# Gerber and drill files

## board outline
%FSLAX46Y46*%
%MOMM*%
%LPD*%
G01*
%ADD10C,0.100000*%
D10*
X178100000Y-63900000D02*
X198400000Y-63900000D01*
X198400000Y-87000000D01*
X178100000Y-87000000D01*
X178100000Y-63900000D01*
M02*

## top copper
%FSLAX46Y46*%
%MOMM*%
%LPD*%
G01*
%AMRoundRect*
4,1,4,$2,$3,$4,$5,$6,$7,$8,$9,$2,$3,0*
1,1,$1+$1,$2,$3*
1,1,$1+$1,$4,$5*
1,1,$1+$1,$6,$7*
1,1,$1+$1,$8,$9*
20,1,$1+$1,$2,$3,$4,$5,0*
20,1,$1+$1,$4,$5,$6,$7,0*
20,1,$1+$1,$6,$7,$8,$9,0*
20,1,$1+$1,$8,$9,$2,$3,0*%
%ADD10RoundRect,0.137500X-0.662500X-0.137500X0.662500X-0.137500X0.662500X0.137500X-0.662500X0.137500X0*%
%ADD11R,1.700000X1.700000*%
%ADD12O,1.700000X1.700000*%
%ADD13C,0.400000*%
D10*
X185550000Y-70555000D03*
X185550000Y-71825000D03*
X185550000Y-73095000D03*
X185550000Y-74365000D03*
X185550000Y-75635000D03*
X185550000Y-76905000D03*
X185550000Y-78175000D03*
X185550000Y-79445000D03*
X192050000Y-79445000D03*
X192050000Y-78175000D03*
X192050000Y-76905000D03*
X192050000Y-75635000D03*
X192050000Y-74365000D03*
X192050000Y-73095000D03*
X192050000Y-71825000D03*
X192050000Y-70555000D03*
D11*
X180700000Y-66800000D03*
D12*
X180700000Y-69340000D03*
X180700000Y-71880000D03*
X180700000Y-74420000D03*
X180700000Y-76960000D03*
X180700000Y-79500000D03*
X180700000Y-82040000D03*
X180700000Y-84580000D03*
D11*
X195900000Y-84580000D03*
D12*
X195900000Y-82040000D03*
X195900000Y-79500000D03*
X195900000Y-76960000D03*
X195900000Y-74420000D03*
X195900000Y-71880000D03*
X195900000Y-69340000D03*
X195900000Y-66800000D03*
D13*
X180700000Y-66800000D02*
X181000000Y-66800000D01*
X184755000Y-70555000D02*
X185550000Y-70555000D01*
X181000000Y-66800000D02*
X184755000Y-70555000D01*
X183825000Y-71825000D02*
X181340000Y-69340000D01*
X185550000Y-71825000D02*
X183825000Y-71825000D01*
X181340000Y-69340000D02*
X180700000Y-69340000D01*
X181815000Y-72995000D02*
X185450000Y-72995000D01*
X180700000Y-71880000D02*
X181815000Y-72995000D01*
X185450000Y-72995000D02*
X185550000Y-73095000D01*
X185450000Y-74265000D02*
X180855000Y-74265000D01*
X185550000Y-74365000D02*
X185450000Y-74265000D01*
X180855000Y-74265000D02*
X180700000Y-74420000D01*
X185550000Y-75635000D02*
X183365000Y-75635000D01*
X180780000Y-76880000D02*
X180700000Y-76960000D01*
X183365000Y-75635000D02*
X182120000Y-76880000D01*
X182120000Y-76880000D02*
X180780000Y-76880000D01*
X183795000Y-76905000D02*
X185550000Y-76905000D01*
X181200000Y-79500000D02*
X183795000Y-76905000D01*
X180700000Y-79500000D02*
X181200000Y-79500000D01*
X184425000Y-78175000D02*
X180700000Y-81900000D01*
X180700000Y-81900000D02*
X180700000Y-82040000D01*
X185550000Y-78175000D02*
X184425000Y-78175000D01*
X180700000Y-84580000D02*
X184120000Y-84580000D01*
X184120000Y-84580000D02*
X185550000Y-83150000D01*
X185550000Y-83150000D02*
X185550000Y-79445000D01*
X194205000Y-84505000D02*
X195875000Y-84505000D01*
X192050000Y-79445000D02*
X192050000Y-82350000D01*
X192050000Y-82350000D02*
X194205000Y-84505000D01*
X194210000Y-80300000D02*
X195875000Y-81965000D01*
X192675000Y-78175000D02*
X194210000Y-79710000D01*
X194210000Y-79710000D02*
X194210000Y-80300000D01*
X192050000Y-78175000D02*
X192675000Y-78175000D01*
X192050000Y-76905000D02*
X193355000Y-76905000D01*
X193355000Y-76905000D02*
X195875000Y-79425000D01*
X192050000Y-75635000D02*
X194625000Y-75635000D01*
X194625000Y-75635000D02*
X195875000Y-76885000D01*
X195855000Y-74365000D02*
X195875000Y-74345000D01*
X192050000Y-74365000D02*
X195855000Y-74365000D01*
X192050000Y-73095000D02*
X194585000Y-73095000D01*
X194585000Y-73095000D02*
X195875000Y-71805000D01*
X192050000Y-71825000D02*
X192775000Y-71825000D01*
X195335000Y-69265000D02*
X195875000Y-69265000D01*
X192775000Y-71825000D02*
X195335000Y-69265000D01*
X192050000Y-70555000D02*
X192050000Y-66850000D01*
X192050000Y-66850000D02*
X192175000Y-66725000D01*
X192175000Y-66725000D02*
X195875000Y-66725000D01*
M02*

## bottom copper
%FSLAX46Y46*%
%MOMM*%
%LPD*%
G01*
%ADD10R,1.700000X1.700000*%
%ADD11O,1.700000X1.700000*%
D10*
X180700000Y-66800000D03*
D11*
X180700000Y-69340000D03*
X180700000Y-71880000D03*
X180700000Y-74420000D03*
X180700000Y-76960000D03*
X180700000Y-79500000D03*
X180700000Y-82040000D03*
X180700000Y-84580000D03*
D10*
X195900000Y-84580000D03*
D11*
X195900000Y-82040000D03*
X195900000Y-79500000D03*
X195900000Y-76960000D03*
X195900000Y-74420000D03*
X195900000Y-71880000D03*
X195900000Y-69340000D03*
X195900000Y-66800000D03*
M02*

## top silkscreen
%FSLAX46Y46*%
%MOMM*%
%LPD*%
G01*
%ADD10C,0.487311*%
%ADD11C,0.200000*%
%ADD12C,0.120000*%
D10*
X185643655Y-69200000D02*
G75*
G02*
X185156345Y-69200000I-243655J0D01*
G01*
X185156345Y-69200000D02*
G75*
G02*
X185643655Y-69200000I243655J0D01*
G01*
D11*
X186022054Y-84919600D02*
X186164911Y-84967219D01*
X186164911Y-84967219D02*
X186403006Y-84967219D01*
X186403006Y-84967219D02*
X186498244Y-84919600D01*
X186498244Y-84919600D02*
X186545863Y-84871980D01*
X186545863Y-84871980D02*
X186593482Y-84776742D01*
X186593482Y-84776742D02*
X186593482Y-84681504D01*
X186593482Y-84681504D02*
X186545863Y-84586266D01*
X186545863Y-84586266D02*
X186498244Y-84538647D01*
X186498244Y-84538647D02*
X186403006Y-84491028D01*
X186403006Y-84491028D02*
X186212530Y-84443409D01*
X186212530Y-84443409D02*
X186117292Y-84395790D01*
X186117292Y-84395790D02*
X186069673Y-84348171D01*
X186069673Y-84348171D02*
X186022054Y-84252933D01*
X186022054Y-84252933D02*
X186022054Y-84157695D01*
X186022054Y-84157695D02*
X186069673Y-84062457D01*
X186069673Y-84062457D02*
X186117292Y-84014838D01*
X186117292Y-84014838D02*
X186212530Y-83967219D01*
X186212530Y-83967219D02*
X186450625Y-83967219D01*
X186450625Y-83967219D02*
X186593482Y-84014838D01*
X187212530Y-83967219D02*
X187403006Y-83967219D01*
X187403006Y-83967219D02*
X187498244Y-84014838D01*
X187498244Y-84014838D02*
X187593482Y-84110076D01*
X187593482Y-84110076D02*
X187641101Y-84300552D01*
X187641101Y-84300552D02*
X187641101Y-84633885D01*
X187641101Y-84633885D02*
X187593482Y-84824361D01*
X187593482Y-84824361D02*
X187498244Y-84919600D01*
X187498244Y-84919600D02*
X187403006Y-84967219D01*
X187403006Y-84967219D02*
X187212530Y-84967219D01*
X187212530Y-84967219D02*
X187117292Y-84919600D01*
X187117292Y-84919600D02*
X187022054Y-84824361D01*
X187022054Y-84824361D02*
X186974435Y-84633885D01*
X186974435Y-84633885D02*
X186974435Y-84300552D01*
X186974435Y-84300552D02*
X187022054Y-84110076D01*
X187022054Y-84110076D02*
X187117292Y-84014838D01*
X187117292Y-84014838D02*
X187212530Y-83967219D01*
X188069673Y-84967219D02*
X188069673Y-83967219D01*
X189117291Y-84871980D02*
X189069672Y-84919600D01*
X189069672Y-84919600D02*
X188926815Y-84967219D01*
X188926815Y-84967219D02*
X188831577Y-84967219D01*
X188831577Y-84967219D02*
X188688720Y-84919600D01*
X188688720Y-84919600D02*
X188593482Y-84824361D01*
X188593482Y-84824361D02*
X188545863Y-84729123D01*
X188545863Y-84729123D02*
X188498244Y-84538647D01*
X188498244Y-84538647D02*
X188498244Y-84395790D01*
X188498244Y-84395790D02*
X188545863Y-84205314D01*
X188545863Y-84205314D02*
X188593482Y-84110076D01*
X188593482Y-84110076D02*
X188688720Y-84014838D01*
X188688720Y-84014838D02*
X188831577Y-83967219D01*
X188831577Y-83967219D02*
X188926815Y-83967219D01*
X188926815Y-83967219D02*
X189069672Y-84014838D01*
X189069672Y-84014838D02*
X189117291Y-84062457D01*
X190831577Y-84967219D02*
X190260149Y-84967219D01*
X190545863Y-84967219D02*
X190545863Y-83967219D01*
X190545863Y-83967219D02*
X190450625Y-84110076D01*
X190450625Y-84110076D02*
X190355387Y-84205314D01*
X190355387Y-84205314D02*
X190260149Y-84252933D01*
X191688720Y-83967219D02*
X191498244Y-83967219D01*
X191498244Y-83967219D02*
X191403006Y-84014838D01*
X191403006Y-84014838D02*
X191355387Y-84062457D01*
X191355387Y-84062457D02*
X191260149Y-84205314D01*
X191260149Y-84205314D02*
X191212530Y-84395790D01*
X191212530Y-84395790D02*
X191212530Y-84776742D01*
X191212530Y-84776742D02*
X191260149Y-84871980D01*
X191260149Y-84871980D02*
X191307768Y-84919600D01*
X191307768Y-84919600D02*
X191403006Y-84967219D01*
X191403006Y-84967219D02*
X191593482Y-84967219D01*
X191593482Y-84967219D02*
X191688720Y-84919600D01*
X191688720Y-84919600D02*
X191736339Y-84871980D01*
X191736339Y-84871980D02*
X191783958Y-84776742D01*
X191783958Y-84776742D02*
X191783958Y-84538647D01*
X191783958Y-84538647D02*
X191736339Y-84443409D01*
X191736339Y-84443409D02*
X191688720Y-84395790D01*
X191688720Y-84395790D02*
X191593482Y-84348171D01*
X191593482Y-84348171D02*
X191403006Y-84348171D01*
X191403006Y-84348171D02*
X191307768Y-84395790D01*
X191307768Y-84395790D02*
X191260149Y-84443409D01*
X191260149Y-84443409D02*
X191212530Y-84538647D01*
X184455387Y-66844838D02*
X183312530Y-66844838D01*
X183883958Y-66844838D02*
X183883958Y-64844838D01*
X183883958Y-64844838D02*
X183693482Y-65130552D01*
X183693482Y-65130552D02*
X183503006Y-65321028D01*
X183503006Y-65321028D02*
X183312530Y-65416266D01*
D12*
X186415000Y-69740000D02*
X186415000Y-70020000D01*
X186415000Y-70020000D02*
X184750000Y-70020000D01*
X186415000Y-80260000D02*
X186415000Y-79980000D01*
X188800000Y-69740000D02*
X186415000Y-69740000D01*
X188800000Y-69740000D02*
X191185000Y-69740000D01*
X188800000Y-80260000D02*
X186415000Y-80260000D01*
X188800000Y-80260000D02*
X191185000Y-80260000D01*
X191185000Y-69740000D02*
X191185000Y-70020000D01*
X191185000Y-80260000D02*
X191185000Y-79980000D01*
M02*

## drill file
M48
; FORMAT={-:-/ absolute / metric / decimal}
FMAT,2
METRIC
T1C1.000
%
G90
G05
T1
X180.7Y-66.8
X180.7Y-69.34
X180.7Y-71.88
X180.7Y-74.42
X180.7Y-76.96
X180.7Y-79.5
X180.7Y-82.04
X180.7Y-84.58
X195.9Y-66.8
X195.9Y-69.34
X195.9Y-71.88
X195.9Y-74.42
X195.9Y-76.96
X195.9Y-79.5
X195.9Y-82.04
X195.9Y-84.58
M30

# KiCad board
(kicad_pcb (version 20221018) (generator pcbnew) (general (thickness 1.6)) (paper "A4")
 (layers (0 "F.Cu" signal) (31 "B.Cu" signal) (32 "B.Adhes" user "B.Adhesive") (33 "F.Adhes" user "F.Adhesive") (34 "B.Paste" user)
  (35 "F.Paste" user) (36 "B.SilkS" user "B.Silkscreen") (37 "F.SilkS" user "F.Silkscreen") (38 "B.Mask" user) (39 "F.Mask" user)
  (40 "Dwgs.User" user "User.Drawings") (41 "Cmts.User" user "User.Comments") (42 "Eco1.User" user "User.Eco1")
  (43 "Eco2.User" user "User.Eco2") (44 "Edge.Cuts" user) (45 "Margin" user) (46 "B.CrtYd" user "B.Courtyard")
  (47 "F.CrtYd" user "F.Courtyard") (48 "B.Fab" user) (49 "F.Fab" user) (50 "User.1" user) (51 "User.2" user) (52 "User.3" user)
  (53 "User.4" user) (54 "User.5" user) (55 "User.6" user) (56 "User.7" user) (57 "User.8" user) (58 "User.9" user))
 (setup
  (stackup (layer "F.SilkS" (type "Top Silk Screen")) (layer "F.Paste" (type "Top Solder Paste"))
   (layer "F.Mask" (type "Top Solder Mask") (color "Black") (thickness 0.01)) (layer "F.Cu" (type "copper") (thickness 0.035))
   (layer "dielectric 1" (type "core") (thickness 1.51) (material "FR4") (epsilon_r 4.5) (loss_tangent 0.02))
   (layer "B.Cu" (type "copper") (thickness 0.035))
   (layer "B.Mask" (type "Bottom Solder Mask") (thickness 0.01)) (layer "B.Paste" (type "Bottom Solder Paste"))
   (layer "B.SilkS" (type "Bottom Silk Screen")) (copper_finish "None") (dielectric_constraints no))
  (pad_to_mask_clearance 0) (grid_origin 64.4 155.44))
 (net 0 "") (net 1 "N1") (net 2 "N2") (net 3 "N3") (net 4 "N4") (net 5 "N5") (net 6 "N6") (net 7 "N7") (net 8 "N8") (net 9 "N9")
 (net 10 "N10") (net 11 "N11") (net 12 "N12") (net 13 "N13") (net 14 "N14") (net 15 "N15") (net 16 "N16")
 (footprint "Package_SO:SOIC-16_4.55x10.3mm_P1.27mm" (layer "F.Cu") (at 188.8 75)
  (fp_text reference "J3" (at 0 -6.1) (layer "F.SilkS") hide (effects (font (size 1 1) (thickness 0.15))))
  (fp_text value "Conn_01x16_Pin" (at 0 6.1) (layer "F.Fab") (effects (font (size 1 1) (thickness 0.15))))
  (fp_line (start -2.385 -5.26) (end -2.385 -4.98) (stroke (width 0.12) (type solid)) (layer "F.SilkS"))
  (fp_line (start -2.385 -4.98) (end -4.05 -4.98) (stroke (width 0.12) (type solid)) (layer "F.SilkS"))
  (fp_line (start -2.385 5.26) (end -2.385 4.98) (stroke (width 0.12) (type solid)) (layer "F.SilkS"))
  (fp_line (start 0 -5.26) (end -2.385 -5.26) (stroke (width 0.12) (type solid)) (layer "F.SilkS"))
  (fp_line (start 0 -5.26) (end 2.385 -5.26) (stroke (width 0.12) (type solid)) (layer "F.SilkS"))
  (fp_line (start 0 5.26) (end -2.385 5.26) (stroke (width 0.12) (type solid)) (layer "F.SilkS"))
  (fp_line (start 0 5.26) (end 2.385 5.26) (stroke (width 0.12) (type solid)) (layer "F.SilkS"))
  (fp_line (start 2.385 -5.26) (end 2.385 -4.98) (stroke (width 0.12) (type solid)) (layer "F.SilkS"))
  (fp_line (start 2.385 5.26) (end 2.385 4.98) (stroke (width 0.12) (type solid)) (layer "F.SilkS"))
  (pad "1" smd roundrect (at -3.25 -4.445) (size 1.6 0.55) (layers "F.Cu" "F.Paste" "F.Mask") (roundrect_rratio 0.25) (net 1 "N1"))
  (pad "2" smd roundrect (at -3.25 -3.175) (size 1.6 0.55) (layers "F.Cu" "F.Paste" "F.Mask") (roundrect_rratio 0.25) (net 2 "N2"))
  (pad "3" smd roundrect (at -3.25 -1.905) (size 1.6 0.55) (layers "F.Cu" "F.Paste" "F.Mask") (roundrect_rratio 0.25) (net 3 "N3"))
  (pad "4" smd roundrect (at -3.25 -0.635) (size 1.6 0.55) (layers "F.Cu" "F.Paste" "F.Mask") (roundrect_rratio 0.25) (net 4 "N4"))
  (pad "5" smd roundrect (at -3.25 0.635) (size 1.6 0.55) (layers "F.Cu" "F.Paste" "F.Mask") (roundrect_rratio 0.25) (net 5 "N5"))
  (pad "6" smd roundrect (at -3.25 1.905) (size 1.6 0.55) (layers "F.Cu" "F.Paste" "F.Mask") (roundrect_rratio 0.25) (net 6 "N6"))
  (pad "7" smd roundrect (at -3.25 3.175) (size 1.6 0.55) (layers "F.Cu" "F.Paste" "F.Mask") (roundrect_rratio 0.25) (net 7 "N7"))
  (pad "8" smd roundrect (at -3.25 4.445) (size 1.6 0.55) (layers "F.Cu" "F.Paste" "F.Mask") (roundrect_rratio 0.25) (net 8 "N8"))
  (pad "9" smd roundrect (at 3.25 4.445) (size 1.6 0.55) (layers "F.Cu" "F.Paste" "F.Mask") (roundrect_rratio 0.25) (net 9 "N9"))
  (pad "10" smd roundrect (at 3.25 3.175) (size 1.6 0.55) (layers "F.Cu" "F.Paste" "F.Mask") (roundrect_rratio 0.25) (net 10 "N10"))
  (pad "11" smd roundrect (at 3.25 1.905) (size 1.6 0.55) (layers "F.Cu" "F.Paste" "F.Mask") (roundrect_rratio 0.25) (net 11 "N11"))
  (pad "12" smd roundrect (at 3.25 0.635) (size 1.6 0.55) (layers "F.Cu" "F.Paste" "F.Mask") (roundrect_rratio 0.25) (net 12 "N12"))
  (pad "13" smd roundrect (at 3.25 -0.635) (size 1.6 0.55) (layers "F.Cu" "F.Paste" "F.Mask") (roundrect_rratio 0.25) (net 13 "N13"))
  (pad "14" smd roundrect (at 3.25 -1.905) (size 1.6 0.55) (layers "F.Cu" "F.Paste" "F.Mask") (roundrect_rratio 0.25) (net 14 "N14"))
  (pad "15" smd roundrect (at 3.25 -3.175) (size 1.6 0.55) (layers "F.Cu" "F.Paste" "F.Mask") (roundrect_rratio 0.25) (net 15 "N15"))
  (pad "16" smd roundrect (at 3.25 -4.445) (size 1.6 0.55) (layers "F.Cu" "F.Paste" "F.Mask") (roundrect_rratio 0.25) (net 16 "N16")))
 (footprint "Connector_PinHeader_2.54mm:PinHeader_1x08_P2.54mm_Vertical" (layer "B.Cu") (at 180.7 66.8 180)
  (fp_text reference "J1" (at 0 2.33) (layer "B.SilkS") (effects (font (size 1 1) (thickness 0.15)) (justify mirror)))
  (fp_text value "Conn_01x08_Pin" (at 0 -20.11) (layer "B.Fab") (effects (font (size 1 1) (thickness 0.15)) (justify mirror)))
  (pad "1" thru_hole rect (at 0 0 180) (size 1.7 1.7) (drill 1) (layers "*.Cu" "*.Mask") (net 1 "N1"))
  (pad "2" thru_hole oval (at 0 -2.54 180) (size 1.7 1.7) (drill 1) (layers "*.Cu" "*.Mask") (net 2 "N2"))
  (pad "3" thru_hole oval (at 0 -5.08 180) (size 1.7 1.7) (drill 1) (layers "*.Cu" "*.Mask") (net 3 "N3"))
  (pad "4" thru_hole oval (at 0 -7.62 180) (size 1.7 1.7) (drill 1) (layers "*.Cu" "*.Mask") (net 4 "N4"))
  (pad "5" thru_hole oval (at 0 -10.16 180) (size 1.7 1.7) (drill 1) (layers "*.Cu" "*.Mask") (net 5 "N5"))
  (pad "6" thru_hole oval (at 0 -12.7 180) (size 1.7 1.7) (drill 1) (layers "*.Cu" "*.Mask") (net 6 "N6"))
  (pad "7" thru_hole oval (at 0 -15.24 180) (size 1.7 1.7) (drill 1) (layers "*.Cu" "*.Mask") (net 7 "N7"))
  (pad "8" thru_hole oval (at 0 -17.78 180) (size 1.7 1.7) (drill 1) (layers "*.Cu" "*.Mask") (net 8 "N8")))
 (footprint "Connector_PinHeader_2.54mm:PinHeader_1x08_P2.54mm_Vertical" (layer "B.Cu") (at 195.9 84.58)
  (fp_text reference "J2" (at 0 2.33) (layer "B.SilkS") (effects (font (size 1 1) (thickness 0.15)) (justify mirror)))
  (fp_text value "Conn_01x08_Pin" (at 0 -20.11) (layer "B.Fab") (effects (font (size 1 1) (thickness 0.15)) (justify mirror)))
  (pad "1" thru_hole rect (at 0 0) (size 1.7 1.7) (drill 1) (layers "*.Cu" "*.Mask") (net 9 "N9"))
  (pad "2" thru_hole oval (at 0 -2.54) (size 1.7 1.7) (drill 1) (layers "*.Cu" "*.Mask") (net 10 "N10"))
  (pad "3" thru_hole oval (at 0 -5.08) (size 1.7 1.7) (drill 1) (layers "*.Cu" "*.Mask") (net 11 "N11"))
  (pad "4" thru_hole oval (at 0 -7.62) (size 1.7 1.7) (drill 1) (layers "*.Cu" "*.Mask") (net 12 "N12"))
  (pad "5" thru_hole oval (at 0 -10.16) (size 1.7 1.7) (drill 1) (layers "*.Cu" "*.Mask") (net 13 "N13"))
  (pad "6" thru_hole oval (at 0 -12.7) (size 1.7 1.7) (drill 1) (layers "*.Cu" "*.Mask") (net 14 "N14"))
  (pad "7" thru_hole oval (at 0 -15.24) (size 1.7 1.7) (drill 1) (layers "*.Cu" "*.Mask") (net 15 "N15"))
  (pad "8" thru_hole oval (at 0 -17.78) (size 1.7 1.7) (drill 1) (layers "*.Cu" "*.Mask") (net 16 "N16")))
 (gr_circle (center 185.4 69.2) (end 185.812311 69.2) (stroke (width 0.15) (type solid)) (fill solid) (layer "F.SilkS"))
 (gr_rect (start 178.1 63.9) (end 198.4 87) (stroke (width 0.1) (type default)) (fill none) (layer "Edge.Cuts"))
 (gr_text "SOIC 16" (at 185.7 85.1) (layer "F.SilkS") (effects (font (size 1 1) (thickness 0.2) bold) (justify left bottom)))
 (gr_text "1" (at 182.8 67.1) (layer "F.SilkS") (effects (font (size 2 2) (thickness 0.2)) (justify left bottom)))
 (segment (start 180.7 66.8) (end 181 66.8) (width 0.4) (layer "F.Cu") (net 1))
 (segment (start 184.755 70.555) (end 185.55 70.555) (width 0.4) (layer "F.Cu") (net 1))
 (segment (start 181 66.8) (end 184.755 70.555) (width 0.4) (layer "F.Cu") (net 1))
 (segment (start 183.825 71.825) (end 181.34 69.34) (width 0.4) (layer "F.Cu") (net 2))
 (segment (start 185.55 71.825) (end 183.825 71.825) (width 0.4) (layer "F.Cu") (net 2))
 (segment (start 181.34 69.34) (end 180.7 69.34) (width 0.4) (layer "F.Cu") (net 2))
 (segment (start 181.815 72.995) (end 185.45 72.995) (width 0.4) (layer "F.Cu") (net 3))
 (segment (start 180.7 71.88) (end 181.815 72.995) (width 0.4) (layer "F.Cu") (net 3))
 (segment (start 185.45 72.995) (end 185.55 73.095) (width 0.4) (layer "F.Cu") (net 3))
 (segment (start 185.45 74.265) (end 180.855 74.265) (width 0.4) (layer "F.Cu") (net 4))
 (segment (start 185.55 74.365) (end 185.45 74.265) (width 0.4) (layer "F.Cu") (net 4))
 (segment (start 180.855 74.265) (end 180.7 74.42) (width 0.4) (layer "F.Cu") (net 4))
 (segment (start 185.55 75.635) (end 183.365 75.635) (width 0.4) (layer "F.Cu") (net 5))
 (segment (start 180.78 76.88) (end 180.7 76.96) (width 0.4) (layer "F.Cu") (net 5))
 (segment (start 183.365 75.635) (end 182.12 76.88) (width 0.4) (layer "F.Cu") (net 5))
 (segment (start 182.12 76.88) (end 180.78 76.88) (width 0.4) (layer "F.Cu") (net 5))
 (segment (start 183.795 76.905) (end 185.55 76.905) (width 0.4) (layer "F.Cu") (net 6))
 (segment (start 181.2 79.5) (end 183.795 76.905) (width 0.4) (layer "F.Cu") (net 6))
 (segment (start 180.7 79.5) (end 181.2 79.5) (width 0.4) (layer "F.Cu") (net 6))
 (segment (start 184.425 78.175) (end 180.7 81.9) (width 0.4) (layer "F.Cu") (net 7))
 (segment (start 180.7 81.9) (end 180.7 82.04) (width 0.4) (layer "F.Cu") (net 7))
 (segment (start 185.55 78.175) (end 184.425 78.175) (width 0.4) (layer "F.Cu") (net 7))
 (segment (start 180.7 84.58) (end 184.12 84.58) (width 0.4) (layer "F.Cu") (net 8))
 (segment (start 184.12 84.58) (end 185.55 83.15) (width 0.4) (layer "F.Cu") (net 8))
 (segment (start 185.55 83.15) (end 185.55 79.445) (width 0.4) (layer "F.Cu") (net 8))
 (segment (start 194.205 84.505) (end 195.875 84.505) (width 0.4) (layer "F.Cu") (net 9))
 (segment (start 192.05 79.445) (end 192.05 82.35) (width 0.4) (layer "F.Cu") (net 9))
 (segment (start 192.05 82.35) (end 194.205 84.505) (width 0.4) (layer "F.Cu") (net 9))
 (segment (start 194.21 80.3) (end 195.875 81.965) (width 0.4) (layer "F.Cu") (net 10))
 (segment (start 192.675 78.175) (end 194.21 79.71) (width 0.4) (layer "F.Cu") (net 10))
 (segment (start 194.21 79.71) (end 194.21 80.3) (width 0.4) (layer "F.Cu") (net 10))
 (segment (start 192.05 78.175) (end 192.675 78.175) (width 0.4) (layer "F.Cu") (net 10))
 (segment (start 192.05 76.905) (end 193.355 76.905) (width 0.4) (layer "F.Cu") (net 11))
 (segment (start 193.355 76.905) (end 195.875 79.425) (width 0.4) (layer "F.Cu") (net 11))
 (segment (start 192.05 75.635) (end 194.625 75.635) (width 0.4) (layer "F.Cu") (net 12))
 (segment (start 194.625 75.635) (end 195.875 76.885) (width 0.4) (layer "F.Cu") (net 12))
 (segment (start 195.855 74.365) (end 195.875 74.345) (width 0.4) (layer "F.Cu") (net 13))
 (segment (start 192.05 74.365) (end 195.855 74.365) (width 0.4) (layer "F.Cu") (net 13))
 (segment (start 192.05 73.095) (end 194.585 73.095) (width 0.4) (layer "F.Cu") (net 14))
 (segment (start 194.585 73.095) (end 195.875 71.805) (width 0.4) (layer "F.Cu") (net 14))
 (segment (start 192.05 71.825) (end 192.775 71.825) (width 0.4) (layer "F.Cu") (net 15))
 (segment (start 195.335 69.265) (end 195.875 69.265) (width 0.4) (layer "F.Cu") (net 15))
 (segment (start 192.775 71.825) (end 195.335 69.265) (width 0.4) (layer "F.Cu") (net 15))
 (segment (start 192.05 70.555) (end 192.05 66.85) (width 0.4) (layer "F.Cu") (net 16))
 (segment (start 192.05 66.85) (end 192.175 66.725) (width 0.4) (layer "F.Cu") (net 16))
 (segment (start 192.175 66.725) (end 195.875 66.725) (width 0.4) (layer "F.Cu") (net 16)))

